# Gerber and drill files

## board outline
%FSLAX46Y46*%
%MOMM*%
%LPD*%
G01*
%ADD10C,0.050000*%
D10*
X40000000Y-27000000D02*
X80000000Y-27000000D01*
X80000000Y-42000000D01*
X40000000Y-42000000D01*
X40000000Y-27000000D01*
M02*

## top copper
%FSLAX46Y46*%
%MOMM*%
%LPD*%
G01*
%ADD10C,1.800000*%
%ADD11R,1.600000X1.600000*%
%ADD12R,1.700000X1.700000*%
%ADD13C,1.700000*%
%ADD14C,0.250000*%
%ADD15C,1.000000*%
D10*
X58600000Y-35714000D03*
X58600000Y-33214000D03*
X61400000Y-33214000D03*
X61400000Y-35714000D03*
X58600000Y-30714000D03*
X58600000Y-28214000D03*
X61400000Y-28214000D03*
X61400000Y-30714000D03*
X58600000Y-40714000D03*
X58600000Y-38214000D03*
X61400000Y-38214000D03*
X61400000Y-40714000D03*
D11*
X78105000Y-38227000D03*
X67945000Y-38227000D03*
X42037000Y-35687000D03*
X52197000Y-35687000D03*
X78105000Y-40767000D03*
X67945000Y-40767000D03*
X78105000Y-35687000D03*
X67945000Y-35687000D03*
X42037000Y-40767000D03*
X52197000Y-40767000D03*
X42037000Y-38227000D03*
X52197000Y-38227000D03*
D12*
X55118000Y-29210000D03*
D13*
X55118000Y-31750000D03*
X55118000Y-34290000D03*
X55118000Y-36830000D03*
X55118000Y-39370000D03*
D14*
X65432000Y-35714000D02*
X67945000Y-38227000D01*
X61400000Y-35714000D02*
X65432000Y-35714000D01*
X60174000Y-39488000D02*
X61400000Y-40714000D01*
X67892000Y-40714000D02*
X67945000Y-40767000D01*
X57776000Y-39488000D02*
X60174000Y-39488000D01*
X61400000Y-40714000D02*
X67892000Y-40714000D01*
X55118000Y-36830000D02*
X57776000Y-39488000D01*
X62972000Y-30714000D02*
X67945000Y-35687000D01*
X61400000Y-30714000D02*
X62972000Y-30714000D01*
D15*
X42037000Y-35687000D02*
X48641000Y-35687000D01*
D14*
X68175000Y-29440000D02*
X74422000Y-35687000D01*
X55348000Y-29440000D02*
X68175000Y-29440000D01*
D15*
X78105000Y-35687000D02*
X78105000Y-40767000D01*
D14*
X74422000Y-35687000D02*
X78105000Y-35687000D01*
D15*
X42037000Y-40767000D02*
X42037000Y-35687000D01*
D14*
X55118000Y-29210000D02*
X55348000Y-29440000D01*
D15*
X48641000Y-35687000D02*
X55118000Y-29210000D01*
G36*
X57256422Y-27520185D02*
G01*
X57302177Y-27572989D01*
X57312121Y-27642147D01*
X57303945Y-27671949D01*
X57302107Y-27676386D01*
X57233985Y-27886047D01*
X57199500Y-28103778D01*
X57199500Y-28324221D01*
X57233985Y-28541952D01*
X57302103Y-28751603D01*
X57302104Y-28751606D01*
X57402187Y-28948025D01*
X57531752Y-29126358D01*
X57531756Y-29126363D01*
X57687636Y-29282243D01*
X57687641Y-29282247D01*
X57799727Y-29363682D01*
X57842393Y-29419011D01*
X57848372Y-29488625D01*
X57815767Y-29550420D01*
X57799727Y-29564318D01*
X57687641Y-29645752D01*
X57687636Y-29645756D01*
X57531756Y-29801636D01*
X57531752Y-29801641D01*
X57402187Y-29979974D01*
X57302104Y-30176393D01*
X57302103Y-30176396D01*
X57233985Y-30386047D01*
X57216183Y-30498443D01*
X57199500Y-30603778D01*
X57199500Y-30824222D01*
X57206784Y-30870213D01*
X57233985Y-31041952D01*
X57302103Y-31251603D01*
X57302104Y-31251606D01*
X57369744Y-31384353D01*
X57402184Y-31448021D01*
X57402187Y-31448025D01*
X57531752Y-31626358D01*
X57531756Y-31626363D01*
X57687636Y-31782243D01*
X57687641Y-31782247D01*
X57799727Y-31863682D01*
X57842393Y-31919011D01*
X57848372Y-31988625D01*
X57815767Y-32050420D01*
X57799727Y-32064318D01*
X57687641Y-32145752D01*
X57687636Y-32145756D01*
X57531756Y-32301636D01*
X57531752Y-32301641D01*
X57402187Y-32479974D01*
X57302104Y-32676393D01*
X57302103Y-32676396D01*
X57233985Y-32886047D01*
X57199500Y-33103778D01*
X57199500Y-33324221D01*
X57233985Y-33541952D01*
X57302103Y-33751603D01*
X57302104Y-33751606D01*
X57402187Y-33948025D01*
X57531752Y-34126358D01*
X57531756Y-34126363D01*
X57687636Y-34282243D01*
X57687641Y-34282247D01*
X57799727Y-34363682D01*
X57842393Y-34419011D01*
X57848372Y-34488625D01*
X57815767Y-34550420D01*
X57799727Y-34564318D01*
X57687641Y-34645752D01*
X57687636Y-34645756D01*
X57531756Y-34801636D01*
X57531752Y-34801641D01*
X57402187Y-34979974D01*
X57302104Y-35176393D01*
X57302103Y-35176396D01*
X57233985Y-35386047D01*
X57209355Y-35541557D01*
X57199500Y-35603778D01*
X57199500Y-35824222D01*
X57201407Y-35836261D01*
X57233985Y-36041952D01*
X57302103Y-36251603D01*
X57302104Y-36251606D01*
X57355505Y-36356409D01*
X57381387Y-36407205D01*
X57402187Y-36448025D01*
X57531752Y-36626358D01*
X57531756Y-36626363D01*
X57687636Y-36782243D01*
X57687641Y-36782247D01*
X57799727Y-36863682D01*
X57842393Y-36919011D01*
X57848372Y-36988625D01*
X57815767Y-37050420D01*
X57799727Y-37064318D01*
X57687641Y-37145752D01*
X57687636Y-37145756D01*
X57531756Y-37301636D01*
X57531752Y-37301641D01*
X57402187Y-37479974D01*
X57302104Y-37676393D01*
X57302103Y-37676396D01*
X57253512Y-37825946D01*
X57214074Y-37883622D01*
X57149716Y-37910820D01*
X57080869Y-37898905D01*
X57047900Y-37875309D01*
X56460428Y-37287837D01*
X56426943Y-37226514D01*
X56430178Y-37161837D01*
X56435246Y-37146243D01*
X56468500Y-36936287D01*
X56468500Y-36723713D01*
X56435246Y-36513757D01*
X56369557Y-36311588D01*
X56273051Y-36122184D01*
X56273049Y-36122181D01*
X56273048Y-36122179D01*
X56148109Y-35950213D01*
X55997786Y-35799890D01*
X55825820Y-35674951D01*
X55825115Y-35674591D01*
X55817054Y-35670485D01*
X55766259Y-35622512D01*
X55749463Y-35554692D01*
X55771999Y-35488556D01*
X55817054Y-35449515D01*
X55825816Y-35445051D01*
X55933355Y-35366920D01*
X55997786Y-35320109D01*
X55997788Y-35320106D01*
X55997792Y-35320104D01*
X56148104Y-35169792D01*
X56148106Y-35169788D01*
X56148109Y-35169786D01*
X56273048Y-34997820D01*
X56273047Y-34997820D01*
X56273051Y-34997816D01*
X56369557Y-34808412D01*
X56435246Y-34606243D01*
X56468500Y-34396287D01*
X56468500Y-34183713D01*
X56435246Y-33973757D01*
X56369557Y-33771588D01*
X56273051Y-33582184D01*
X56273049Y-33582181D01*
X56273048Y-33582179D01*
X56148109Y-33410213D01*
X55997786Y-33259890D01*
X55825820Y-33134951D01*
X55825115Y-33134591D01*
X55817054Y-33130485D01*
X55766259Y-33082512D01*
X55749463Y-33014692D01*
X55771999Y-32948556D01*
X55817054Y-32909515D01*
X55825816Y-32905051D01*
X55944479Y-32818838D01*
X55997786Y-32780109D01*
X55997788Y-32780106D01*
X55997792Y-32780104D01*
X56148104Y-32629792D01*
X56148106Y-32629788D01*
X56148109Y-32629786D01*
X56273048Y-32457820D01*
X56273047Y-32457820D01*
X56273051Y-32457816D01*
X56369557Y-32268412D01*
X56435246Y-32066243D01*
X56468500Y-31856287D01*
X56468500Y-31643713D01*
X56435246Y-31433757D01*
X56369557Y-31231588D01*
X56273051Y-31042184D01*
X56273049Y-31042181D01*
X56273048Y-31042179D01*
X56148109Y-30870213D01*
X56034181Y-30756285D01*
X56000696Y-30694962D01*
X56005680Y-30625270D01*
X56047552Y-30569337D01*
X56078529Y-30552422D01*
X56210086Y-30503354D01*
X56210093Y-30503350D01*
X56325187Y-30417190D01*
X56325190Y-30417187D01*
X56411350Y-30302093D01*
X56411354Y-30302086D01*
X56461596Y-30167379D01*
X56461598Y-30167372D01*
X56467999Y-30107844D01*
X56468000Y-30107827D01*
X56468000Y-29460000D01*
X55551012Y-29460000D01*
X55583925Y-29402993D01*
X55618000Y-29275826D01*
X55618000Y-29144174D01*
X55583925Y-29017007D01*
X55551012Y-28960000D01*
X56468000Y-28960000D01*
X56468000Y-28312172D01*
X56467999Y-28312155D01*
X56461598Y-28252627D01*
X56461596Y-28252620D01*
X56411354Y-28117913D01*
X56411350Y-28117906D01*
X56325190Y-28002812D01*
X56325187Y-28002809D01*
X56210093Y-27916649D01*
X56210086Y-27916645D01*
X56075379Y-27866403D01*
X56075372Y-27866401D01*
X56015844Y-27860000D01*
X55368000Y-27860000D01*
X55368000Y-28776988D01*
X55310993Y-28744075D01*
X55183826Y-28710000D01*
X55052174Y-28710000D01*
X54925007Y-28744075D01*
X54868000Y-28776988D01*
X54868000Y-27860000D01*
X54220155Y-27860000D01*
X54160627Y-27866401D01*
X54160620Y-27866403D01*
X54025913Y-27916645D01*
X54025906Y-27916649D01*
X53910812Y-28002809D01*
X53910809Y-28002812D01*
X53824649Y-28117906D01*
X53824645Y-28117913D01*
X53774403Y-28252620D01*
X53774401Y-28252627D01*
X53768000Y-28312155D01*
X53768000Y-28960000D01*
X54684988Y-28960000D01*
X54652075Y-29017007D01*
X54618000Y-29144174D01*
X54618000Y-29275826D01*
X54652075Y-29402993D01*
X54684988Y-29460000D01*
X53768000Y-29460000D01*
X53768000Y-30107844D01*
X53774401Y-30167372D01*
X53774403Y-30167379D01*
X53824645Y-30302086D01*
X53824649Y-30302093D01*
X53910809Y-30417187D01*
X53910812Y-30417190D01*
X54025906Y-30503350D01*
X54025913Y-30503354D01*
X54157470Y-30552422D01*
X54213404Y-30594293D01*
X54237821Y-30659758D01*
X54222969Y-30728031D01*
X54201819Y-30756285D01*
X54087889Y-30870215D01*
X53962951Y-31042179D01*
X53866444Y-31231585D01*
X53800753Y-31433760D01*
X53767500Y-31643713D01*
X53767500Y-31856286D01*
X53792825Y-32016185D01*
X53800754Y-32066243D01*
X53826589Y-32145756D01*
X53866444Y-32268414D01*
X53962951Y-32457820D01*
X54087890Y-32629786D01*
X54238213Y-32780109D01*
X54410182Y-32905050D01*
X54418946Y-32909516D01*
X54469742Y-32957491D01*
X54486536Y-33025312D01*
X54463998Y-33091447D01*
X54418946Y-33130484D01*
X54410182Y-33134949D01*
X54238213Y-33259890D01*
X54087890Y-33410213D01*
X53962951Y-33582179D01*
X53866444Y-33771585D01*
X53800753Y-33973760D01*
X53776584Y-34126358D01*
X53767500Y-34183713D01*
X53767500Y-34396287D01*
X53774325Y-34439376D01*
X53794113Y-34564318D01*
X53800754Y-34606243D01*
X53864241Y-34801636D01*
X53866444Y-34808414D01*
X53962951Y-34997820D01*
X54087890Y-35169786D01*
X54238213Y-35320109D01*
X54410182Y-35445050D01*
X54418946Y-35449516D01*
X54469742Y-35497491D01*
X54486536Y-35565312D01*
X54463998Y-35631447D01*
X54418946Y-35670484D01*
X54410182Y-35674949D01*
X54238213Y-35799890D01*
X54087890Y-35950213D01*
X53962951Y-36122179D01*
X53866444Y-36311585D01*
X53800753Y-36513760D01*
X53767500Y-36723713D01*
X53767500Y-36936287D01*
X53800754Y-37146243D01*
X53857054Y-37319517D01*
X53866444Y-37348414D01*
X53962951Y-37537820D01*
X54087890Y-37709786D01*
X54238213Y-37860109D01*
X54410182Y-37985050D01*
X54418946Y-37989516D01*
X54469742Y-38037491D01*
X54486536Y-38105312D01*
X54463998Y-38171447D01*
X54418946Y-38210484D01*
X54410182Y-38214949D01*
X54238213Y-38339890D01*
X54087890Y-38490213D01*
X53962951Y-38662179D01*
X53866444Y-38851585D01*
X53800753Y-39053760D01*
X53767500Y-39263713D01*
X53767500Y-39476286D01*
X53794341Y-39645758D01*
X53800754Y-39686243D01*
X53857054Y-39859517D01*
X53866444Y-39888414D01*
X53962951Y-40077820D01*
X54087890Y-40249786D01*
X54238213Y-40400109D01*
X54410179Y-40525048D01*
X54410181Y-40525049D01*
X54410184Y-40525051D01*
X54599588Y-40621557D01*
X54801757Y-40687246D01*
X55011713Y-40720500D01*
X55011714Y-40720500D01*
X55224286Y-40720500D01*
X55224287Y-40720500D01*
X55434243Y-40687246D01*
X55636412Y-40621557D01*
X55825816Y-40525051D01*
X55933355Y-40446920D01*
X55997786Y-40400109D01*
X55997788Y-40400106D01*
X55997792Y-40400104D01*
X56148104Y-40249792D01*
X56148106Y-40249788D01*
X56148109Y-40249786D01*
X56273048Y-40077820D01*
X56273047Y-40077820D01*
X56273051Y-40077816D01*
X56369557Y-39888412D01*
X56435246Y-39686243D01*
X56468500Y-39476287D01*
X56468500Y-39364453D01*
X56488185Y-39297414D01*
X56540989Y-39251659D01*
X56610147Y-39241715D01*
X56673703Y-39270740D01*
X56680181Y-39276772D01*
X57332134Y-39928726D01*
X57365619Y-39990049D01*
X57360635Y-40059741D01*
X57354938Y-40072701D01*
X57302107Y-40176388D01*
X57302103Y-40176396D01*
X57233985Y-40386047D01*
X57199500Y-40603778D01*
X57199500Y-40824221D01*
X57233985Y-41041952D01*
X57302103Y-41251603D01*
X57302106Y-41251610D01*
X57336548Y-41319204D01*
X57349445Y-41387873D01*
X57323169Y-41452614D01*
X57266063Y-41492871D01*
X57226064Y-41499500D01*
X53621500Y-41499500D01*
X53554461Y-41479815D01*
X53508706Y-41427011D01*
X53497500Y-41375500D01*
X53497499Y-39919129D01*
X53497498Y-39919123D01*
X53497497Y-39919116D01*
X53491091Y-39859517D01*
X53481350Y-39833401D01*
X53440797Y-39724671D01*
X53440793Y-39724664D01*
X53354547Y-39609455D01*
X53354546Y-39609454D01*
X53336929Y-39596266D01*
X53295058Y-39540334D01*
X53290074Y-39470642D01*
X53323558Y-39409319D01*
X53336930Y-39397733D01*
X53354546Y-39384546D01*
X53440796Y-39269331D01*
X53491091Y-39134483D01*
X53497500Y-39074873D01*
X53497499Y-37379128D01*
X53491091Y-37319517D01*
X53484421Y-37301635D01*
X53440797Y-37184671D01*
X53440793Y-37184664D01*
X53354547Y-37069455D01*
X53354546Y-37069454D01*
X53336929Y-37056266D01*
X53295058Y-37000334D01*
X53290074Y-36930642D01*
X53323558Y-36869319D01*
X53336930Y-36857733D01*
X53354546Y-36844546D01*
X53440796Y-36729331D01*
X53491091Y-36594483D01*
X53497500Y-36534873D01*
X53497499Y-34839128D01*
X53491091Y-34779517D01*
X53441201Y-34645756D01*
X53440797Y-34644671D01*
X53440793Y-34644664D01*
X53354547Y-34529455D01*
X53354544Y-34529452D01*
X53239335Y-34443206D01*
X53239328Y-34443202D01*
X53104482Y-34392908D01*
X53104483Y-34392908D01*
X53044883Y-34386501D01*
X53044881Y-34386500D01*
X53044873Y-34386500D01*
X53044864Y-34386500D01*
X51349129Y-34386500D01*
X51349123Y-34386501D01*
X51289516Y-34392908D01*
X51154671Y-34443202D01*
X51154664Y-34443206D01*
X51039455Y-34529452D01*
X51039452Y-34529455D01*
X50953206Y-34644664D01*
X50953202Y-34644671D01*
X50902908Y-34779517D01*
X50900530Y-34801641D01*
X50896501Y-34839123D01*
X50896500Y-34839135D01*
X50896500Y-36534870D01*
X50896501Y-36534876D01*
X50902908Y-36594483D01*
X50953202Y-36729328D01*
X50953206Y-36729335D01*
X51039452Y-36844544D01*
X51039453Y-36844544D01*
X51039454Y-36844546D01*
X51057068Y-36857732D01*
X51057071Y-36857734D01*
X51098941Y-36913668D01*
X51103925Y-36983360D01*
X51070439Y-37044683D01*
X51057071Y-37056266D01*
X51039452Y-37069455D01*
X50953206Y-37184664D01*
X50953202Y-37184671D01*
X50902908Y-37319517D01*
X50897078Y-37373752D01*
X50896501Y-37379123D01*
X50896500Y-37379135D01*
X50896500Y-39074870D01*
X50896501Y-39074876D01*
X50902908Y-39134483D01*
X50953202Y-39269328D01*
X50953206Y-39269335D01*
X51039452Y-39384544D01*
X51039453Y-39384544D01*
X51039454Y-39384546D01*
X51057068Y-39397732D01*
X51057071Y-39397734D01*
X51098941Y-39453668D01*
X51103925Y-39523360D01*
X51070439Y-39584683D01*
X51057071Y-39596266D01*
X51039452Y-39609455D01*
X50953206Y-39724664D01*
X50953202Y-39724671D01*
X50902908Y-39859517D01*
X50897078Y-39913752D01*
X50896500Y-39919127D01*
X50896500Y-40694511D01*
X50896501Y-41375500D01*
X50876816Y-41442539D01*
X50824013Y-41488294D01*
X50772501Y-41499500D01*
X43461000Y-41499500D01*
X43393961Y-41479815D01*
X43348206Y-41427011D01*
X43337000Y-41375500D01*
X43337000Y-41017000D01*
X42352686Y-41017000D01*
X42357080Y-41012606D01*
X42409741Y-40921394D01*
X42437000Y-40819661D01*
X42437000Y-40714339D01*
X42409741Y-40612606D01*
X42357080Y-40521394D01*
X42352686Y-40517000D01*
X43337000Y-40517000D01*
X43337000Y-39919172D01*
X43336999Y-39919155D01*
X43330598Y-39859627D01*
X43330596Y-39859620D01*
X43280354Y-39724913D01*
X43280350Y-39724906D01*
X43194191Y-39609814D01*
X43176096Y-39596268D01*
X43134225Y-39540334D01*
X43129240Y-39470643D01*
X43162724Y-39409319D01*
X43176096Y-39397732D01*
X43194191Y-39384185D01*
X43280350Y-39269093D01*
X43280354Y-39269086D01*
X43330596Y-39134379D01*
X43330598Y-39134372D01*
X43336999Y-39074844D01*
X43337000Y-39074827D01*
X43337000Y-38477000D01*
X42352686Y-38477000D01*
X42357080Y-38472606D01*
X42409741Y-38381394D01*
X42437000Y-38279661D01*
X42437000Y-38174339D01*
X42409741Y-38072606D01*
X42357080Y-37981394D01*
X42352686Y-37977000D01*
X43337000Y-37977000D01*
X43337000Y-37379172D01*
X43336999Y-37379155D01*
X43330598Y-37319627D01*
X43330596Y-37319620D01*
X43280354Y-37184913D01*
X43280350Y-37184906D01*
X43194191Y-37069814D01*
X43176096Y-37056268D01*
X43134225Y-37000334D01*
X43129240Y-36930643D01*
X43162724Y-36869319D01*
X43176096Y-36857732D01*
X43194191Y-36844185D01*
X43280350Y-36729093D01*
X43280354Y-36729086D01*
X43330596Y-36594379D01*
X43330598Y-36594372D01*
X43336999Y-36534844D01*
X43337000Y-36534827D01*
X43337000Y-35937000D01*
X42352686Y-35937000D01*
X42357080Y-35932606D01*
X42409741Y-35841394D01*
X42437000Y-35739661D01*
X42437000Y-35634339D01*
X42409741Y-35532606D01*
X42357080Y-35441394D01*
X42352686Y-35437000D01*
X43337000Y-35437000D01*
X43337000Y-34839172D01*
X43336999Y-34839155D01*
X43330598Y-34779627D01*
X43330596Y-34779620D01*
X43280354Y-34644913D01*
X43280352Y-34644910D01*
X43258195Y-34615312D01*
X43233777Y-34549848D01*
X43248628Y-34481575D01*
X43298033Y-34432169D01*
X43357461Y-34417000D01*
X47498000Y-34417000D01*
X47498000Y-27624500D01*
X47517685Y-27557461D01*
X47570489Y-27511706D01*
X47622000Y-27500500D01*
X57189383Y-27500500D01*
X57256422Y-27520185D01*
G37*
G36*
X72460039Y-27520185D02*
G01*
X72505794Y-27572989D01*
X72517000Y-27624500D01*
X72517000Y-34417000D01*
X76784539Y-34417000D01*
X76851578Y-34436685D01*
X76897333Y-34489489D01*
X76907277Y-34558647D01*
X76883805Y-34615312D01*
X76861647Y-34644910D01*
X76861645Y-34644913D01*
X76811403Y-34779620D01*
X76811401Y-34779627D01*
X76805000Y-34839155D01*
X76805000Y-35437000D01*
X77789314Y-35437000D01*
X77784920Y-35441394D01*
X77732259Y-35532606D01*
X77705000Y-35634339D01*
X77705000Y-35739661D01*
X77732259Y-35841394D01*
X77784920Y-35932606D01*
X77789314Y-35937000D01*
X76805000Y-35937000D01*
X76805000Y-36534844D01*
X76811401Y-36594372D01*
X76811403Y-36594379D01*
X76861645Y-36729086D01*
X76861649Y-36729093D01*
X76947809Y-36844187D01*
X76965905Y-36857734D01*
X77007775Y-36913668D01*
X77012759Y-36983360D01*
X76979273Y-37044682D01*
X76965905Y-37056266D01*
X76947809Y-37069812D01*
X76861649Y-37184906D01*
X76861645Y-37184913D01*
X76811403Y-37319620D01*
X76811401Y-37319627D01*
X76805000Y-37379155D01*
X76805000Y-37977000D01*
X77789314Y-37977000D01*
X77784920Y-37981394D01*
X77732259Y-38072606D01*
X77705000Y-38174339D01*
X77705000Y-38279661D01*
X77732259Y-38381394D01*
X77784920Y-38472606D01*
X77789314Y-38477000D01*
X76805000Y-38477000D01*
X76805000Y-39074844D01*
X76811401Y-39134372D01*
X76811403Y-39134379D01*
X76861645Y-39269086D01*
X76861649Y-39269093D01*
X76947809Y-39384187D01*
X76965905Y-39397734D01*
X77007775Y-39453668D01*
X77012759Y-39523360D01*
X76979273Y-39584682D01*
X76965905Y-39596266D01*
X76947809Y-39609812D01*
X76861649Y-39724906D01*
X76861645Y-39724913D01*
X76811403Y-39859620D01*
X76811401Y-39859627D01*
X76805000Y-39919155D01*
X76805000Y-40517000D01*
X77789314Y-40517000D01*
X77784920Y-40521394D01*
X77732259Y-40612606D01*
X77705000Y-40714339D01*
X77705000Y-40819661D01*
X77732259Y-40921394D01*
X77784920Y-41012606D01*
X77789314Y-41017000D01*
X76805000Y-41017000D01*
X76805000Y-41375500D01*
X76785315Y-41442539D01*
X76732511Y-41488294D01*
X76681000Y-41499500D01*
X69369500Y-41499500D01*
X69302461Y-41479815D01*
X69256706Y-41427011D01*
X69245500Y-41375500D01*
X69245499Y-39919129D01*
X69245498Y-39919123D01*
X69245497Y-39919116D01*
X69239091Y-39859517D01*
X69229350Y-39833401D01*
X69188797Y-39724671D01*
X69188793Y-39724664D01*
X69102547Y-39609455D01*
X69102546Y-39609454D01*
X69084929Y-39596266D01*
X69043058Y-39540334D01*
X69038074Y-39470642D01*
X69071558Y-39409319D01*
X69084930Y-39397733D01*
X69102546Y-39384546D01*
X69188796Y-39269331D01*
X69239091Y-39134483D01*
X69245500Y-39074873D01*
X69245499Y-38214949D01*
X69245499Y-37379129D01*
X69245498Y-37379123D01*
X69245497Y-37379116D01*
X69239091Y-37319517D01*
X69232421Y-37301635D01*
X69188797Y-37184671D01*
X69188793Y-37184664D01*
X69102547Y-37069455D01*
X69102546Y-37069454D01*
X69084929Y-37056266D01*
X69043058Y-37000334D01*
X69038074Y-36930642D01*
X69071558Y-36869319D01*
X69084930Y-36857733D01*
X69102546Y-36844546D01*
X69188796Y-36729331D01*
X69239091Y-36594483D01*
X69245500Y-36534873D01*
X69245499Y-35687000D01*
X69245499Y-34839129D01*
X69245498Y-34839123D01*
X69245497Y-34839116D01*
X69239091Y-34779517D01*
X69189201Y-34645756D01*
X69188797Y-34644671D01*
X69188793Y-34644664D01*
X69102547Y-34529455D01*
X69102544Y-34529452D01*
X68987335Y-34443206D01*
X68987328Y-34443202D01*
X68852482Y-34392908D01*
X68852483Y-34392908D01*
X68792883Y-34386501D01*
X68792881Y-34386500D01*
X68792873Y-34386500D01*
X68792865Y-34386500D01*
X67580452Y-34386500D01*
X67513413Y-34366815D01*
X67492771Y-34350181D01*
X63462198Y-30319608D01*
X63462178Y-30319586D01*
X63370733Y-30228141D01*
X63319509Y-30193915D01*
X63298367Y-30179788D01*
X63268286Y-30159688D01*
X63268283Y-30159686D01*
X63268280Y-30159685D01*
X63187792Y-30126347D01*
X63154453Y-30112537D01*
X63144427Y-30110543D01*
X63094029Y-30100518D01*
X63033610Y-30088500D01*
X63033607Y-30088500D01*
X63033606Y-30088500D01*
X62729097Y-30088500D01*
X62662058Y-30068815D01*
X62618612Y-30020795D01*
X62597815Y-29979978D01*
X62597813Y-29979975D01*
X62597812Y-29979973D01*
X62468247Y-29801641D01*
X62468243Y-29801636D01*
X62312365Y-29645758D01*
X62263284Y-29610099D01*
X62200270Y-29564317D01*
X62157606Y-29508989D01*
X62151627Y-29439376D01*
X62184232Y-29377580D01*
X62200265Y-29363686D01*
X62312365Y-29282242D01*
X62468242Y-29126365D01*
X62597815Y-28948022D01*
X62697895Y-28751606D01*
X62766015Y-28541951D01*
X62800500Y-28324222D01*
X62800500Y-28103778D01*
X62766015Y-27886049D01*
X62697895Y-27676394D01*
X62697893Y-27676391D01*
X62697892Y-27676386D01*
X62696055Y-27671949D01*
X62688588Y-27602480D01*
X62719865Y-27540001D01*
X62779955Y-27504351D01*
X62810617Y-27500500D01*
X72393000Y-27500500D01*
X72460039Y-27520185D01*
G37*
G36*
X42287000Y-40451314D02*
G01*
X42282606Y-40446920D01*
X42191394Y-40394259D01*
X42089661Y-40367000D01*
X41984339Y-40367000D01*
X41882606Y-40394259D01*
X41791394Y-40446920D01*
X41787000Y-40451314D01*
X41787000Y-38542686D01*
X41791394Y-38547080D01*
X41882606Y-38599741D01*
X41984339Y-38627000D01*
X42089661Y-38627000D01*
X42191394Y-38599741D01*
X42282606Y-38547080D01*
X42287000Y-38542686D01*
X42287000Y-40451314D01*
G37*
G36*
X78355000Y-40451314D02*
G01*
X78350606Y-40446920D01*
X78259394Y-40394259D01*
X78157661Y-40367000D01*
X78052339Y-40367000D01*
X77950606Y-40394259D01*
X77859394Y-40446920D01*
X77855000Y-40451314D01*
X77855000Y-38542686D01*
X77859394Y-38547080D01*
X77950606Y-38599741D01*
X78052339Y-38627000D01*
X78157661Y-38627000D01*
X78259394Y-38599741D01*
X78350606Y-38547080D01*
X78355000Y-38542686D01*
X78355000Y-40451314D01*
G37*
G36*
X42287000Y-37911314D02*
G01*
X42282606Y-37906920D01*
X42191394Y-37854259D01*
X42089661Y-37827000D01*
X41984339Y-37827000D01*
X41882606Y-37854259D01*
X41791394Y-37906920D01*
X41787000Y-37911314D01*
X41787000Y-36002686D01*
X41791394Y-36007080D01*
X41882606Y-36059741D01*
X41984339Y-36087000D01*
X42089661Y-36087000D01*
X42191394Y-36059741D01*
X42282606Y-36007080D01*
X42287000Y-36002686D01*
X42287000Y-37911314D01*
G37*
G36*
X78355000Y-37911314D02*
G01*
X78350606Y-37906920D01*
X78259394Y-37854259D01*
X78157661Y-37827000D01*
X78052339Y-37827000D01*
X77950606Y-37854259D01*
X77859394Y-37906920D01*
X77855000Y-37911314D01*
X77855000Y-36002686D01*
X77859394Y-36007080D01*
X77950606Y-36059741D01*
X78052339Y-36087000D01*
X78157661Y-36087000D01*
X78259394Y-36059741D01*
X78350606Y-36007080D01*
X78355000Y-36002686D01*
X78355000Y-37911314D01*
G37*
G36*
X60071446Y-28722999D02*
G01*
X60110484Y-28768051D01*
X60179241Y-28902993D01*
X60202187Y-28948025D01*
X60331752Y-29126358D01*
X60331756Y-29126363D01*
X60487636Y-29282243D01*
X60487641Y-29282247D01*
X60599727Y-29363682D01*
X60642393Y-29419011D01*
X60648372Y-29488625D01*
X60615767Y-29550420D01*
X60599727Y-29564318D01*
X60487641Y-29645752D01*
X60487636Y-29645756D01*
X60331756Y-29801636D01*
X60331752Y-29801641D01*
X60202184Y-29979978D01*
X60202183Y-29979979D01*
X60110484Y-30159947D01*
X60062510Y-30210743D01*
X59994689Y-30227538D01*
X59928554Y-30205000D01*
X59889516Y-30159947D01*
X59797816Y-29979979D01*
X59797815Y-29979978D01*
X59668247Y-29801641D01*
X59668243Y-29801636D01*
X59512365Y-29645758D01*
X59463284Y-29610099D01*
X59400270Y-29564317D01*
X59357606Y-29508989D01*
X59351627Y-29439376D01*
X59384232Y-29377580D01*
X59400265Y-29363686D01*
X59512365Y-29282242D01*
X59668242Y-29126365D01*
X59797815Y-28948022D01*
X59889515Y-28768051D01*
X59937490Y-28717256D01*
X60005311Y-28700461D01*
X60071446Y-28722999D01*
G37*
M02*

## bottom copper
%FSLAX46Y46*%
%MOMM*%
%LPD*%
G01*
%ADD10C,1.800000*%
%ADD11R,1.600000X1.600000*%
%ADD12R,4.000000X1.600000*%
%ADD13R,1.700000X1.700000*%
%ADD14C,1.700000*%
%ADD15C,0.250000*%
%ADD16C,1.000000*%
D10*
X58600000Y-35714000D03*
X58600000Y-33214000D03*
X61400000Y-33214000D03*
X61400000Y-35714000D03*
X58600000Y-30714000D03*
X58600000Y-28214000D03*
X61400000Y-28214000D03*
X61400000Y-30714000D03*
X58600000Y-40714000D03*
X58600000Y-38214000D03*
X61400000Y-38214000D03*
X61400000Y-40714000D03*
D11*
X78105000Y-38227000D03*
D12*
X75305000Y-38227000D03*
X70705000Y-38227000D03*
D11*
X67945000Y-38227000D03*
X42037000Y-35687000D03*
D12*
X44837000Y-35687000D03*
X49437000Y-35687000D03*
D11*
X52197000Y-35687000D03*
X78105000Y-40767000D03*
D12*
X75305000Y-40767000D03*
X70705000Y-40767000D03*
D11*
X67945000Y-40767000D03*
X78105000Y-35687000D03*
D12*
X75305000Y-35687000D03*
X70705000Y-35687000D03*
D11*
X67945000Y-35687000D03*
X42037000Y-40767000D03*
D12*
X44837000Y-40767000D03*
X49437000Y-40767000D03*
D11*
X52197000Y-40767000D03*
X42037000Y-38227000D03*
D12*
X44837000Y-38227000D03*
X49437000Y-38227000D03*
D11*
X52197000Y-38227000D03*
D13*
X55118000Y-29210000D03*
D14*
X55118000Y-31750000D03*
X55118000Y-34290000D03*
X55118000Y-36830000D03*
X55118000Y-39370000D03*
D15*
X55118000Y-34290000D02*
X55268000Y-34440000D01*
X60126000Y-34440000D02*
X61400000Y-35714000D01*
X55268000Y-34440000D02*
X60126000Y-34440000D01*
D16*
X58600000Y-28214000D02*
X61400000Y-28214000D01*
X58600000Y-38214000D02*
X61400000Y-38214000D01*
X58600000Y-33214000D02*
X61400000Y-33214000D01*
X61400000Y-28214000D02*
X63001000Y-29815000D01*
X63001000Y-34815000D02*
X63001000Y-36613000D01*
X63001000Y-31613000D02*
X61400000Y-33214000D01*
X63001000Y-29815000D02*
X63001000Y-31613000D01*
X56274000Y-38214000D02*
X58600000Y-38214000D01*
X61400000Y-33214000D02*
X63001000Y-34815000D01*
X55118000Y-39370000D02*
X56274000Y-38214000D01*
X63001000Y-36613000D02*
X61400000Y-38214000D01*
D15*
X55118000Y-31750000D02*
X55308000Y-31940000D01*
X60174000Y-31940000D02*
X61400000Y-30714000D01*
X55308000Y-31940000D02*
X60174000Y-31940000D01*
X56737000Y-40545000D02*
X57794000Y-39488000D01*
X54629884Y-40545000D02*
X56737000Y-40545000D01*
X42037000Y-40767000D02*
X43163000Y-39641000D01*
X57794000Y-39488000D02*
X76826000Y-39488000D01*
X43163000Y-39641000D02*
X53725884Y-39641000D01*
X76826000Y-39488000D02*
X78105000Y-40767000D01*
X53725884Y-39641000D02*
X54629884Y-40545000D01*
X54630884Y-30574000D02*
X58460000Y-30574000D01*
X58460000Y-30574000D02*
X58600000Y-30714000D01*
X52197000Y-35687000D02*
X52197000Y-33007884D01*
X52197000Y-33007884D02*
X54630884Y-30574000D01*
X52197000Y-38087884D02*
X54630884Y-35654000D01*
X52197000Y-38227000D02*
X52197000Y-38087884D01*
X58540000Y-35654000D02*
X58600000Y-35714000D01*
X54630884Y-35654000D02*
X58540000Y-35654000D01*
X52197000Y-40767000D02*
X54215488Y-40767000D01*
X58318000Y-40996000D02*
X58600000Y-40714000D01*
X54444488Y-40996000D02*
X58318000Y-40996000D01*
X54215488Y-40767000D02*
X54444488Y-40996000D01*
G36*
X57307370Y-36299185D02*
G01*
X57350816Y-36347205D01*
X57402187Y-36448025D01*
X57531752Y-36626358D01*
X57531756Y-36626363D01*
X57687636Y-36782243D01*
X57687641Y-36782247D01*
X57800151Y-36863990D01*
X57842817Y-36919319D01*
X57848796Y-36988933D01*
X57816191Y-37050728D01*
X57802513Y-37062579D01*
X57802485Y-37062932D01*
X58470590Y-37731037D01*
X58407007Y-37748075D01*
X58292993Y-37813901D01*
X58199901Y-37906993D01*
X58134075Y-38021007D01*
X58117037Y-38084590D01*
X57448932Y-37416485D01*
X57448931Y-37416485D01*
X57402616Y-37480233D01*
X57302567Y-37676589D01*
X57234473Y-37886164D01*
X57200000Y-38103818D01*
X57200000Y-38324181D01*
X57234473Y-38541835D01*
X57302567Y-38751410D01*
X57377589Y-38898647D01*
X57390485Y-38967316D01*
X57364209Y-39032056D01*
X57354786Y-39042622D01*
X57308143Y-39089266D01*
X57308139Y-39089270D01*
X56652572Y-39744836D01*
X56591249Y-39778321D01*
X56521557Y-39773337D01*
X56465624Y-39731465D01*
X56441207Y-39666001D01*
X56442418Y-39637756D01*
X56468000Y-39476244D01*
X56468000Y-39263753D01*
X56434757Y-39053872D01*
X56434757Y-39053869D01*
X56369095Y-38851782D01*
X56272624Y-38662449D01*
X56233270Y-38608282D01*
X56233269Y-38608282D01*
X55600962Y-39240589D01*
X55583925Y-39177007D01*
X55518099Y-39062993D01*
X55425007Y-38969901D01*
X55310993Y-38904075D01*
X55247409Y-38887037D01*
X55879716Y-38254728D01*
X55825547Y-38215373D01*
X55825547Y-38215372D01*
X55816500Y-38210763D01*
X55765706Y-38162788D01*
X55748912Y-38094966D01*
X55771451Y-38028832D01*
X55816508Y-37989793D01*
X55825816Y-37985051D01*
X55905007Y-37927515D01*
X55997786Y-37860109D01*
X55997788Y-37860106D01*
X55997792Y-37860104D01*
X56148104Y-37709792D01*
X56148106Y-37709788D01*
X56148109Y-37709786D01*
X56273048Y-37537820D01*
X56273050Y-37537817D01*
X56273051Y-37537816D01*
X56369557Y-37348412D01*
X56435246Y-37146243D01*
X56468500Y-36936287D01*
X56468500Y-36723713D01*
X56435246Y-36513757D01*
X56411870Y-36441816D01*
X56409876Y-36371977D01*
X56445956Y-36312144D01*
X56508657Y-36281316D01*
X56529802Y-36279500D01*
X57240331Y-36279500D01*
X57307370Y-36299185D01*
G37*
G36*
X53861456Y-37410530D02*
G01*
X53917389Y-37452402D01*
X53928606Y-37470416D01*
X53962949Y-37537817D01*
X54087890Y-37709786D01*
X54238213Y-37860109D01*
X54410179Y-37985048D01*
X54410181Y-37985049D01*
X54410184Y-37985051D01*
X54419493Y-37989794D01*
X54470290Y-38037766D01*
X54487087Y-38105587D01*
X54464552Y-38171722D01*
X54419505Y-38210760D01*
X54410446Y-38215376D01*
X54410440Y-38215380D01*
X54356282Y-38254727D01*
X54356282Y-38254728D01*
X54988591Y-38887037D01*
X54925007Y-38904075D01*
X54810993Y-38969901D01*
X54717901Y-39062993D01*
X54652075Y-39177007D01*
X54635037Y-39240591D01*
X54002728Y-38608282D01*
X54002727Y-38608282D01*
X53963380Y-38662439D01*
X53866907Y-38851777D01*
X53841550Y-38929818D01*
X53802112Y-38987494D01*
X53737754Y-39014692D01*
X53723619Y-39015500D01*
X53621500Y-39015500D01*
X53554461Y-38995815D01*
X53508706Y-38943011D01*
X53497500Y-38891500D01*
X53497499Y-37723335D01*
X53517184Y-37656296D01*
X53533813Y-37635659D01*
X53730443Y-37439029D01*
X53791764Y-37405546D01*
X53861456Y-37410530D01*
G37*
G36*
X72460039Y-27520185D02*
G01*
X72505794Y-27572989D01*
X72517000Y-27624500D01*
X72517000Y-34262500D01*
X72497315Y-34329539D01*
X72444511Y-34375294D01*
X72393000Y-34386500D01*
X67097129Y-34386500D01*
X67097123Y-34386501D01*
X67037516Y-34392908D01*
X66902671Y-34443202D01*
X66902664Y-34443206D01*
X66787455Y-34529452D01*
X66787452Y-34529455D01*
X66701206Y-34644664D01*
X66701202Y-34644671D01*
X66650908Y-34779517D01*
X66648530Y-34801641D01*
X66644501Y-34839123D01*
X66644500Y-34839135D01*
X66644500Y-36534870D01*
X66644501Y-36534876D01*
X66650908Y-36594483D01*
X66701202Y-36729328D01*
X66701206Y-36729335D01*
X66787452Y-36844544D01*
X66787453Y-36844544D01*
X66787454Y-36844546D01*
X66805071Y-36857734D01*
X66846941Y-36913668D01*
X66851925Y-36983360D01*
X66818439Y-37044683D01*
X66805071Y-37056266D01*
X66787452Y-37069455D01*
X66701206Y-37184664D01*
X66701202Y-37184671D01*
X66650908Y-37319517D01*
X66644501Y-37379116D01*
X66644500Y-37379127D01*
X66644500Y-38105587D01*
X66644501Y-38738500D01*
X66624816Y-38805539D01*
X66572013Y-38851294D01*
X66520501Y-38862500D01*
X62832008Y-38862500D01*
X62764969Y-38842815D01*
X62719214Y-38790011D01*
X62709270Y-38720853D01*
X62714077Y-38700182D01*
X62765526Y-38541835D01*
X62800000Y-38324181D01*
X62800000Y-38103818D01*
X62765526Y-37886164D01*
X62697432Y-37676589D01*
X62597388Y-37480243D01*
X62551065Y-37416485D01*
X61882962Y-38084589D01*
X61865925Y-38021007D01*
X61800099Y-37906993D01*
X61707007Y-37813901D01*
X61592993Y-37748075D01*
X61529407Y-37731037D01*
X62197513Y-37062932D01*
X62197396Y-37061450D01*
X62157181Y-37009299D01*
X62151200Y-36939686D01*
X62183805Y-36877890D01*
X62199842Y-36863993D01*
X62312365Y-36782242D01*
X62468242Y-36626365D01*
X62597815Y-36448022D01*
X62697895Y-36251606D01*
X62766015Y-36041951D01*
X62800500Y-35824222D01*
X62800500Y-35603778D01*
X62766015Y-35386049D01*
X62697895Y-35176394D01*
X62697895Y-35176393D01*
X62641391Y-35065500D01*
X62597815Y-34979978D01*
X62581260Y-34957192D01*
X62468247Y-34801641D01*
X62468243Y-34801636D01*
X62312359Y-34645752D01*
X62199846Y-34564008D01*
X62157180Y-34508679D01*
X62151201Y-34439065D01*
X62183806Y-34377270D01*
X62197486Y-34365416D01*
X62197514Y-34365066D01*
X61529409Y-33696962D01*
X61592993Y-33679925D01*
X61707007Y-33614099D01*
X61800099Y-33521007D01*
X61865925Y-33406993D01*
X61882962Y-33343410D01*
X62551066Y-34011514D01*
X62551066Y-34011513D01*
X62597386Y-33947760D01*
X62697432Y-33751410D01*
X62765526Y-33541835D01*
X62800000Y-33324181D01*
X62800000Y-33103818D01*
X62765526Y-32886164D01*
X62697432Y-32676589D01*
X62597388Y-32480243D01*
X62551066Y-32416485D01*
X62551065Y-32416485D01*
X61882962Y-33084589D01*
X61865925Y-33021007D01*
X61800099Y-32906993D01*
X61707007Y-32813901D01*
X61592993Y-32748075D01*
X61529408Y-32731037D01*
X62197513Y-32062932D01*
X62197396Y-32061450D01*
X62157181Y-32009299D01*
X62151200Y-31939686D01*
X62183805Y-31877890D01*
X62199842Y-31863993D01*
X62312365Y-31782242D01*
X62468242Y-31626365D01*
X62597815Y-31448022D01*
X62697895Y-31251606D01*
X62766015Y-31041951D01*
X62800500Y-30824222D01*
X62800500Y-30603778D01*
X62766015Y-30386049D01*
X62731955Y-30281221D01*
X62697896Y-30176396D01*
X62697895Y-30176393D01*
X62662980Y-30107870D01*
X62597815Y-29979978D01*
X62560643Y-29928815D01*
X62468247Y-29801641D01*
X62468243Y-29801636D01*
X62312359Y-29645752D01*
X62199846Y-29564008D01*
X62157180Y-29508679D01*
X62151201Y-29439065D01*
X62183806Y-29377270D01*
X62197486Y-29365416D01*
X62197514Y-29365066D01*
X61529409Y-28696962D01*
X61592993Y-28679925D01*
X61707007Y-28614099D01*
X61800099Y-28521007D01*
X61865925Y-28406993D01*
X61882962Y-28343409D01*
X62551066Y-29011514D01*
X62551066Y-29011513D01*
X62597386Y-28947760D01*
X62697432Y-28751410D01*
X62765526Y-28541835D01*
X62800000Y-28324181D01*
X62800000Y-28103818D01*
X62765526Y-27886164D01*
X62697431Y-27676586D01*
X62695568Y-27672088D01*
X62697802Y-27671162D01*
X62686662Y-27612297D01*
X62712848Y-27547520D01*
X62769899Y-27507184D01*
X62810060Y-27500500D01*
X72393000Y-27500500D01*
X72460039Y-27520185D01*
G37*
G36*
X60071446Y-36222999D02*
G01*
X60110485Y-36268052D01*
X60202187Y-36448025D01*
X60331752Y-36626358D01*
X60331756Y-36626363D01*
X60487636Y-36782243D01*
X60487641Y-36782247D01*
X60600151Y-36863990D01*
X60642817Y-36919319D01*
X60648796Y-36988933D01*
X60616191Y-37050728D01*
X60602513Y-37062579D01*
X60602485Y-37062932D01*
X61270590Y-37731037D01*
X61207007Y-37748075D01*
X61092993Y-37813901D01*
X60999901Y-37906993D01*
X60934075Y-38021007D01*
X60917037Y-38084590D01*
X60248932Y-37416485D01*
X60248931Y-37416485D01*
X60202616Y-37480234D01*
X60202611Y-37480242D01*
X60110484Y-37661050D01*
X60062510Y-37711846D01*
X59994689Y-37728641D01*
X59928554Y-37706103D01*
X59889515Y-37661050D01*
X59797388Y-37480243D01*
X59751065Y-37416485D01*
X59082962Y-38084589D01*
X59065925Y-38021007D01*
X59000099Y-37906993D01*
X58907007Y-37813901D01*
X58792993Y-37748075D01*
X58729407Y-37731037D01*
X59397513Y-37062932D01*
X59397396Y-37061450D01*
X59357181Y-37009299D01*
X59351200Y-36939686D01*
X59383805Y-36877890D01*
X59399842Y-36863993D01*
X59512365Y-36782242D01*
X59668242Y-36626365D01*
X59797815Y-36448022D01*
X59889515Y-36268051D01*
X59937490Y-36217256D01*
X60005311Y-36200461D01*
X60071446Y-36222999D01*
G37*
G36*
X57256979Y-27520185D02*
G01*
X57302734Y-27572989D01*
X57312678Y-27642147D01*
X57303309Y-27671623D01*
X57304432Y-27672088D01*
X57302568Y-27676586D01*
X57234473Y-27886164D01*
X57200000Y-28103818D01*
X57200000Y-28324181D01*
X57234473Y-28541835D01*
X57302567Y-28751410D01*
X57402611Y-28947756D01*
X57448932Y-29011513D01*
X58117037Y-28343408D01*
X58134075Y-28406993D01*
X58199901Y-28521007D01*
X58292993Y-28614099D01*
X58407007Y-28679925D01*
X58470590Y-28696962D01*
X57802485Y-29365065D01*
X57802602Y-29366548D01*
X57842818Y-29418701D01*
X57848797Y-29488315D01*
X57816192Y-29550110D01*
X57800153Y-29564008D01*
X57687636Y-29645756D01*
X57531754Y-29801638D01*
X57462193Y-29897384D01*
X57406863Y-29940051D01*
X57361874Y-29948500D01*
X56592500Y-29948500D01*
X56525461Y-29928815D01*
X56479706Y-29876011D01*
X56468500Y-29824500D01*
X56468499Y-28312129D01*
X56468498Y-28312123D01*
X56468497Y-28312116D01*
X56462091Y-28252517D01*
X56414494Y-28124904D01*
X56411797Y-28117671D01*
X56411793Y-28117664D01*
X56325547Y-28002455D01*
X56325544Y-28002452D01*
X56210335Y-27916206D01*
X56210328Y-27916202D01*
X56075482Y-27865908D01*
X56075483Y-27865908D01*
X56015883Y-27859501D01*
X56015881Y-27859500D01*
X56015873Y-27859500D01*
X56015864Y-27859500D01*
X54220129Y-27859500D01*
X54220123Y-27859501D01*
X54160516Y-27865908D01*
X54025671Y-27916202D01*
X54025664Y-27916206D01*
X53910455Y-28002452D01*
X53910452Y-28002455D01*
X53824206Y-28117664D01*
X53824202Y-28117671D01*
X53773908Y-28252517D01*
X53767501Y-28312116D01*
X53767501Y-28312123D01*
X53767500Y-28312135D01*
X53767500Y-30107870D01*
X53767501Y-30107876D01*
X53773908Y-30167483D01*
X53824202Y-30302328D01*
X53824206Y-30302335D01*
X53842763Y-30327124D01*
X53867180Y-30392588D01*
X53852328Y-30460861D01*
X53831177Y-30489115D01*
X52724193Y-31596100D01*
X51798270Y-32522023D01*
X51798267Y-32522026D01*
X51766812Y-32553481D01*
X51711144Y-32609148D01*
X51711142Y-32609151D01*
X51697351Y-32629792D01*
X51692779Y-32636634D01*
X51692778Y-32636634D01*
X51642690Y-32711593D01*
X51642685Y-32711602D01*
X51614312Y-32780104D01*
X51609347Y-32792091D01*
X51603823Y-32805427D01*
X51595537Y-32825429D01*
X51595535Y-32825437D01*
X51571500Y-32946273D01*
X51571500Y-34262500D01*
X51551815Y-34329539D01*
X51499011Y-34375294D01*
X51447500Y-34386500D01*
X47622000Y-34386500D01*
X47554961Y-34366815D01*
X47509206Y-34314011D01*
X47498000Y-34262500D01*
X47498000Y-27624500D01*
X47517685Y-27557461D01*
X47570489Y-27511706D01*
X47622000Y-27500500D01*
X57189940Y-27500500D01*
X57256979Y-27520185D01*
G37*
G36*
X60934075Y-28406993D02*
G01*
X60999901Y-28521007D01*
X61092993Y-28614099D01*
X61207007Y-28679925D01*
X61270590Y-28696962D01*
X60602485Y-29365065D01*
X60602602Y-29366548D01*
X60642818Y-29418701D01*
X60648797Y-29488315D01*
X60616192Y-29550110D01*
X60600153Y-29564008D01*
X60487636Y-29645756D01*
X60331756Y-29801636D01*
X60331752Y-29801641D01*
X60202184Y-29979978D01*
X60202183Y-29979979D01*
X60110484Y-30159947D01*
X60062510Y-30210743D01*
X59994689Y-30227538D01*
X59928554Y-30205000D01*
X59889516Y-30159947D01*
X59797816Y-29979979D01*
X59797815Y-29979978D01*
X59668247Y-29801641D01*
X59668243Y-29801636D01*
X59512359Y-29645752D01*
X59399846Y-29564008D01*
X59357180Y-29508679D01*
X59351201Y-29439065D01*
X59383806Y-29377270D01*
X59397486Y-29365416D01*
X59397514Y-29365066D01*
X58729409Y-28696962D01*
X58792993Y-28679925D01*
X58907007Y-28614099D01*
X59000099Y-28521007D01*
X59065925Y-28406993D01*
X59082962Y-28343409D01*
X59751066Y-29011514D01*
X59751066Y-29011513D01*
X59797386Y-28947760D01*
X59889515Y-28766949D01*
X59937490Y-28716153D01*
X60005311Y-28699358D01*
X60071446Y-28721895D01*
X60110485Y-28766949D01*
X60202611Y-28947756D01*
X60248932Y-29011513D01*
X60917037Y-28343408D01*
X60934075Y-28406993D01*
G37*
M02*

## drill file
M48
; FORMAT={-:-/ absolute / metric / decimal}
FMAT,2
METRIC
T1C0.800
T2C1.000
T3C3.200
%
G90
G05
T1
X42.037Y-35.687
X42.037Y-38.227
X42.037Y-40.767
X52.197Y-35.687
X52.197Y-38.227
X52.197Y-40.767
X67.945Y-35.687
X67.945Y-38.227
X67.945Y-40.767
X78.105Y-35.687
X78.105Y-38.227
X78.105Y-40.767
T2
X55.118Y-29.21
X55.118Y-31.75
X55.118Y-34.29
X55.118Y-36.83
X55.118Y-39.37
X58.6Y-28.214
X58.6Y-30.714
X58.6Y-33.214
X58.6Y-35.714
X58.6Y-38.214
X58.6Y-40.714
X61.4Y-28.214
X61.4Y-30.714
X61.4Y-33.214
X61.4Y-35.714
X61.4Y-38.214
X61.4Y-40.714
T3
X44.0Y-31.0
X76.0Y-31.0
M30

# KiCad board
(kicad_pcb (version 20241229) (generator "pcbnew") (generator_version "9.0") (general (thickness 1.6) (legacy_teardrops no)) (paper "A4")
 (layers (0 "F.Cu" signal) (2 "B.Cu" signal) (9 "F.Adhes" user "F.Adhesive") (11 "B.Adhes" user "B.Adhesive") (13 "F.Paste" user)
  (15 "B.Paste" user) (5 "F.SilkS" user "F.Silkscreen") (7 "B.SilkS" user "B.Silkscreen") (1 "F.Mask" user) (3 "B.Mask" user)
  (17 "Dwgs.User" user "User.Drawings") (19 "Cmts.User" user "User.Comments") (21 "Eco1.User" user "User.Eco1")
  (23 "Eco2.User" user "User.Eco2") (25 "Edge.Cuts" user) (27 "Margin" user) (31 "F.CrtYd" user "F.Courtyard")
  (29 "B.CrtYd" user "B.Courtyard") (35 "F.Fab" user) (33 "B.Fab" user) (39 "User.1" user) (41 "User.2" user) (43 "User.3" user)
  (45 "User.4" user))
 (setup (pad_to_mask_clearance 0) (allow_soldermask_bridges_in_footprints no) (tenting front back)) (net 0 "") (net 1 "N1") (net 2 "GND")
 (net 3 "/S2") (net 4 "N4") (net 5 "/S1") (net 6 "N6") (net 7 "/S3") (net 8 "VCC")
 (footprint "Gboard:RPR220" (layer "F.Cu") (at 60 34.464)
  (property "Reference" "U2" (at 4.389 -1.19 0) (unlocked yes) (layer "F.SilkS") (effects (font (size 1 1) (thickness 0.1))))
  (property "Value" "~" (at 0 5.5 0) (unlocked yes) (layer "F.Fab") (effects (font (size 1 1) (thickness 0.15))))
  (pad "1" thru_hole circle (at -1.4 1.25) (size 1.8 1.8) (drill 1) (layers "*.Cu" "*.Mask") (remove_unused_layers no) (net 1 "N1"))
  (pad "2" thru_hole circle (at -1.4 -1.25) (size 1.8 1.8) (drill 1) (layers "*.Cu" "*.Mask") (remove_unused_layers no) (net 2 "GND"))
  (pad "3" thru_hole circle (at 1.4 -1.25) (size 1.8 1.8) (drill 1) (layers "*.Cu" "*.Mask") (remove_unused_layers no) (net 2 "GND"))
  (pad "4" thru_hole circle (at 1.4 1.25) (size 1.8 1.8) (drill 1) (layers "*.Cu" "*.Mask") (remove_unused_layers no) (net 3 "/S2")))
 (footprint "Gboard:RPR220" (layer "F.Cu") (at 60 29.464)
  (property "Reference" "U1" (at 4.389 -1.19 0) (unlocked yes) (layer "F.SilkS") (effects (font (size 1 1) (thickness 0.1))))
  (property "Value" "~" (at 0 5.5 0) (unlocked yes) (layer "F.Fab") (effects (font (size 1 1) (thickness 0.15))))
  (pad "1" thru_hole circle (at -1.4 1.25) (size 1.8 1.8) (drill 1) (layers "*.Cu" "*.Mask") (remove_unused_layers no) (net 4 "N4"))
  (pad "2" thru_hole circle (at -1.4 -1.25) (size 1.8 1.8) (drill 1) (layers "*.Cu" "*.Mask") (remove_unused_layers no) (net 2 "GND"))
  (pad "3" thru_hole circle (at 1.4 -1.25) (size 1.8 1.8) (drill 1) (layers "*.Cu" "*.Mask") (remove_unused_layers no) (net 2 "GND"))
  (pad "4" thru_hole circle (at 1.4 1.25) (size 1.8 1.8) (drill 1) (layers "*.Cu" "*.Mask") (remove_unused_layers no) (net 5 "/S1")))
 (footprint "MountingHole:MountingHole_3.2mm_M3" (layer "F.Cu") (at 76 31)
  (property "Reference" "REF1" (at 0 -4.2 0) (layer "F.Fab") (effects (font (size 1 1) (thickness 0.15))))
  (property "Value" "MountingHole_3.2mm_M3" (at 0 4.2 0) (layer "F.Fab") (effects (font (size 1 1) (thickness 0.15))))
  (pad "" np_thru_hole circle (at 0 0) (size 3.2 3.2) (drill 3.2) (layers "*.Cu" "*.Mask")))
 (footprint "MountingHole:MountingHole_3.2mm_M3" (layer "F.Cu") (at 44 31)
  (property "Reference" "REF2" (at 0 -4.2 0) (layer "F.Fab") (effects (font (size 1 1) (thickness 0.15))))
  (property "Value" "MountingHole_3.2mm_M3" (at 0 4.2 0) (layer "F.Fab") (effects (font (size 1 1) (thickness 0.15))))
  (pad "" np_thru_hole circle (at 0 0) (size 3.2 3.2) (drill 3.2) (layers "*.Cu" "*.Mask")))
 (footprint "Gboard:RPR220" (layer "F.Cu") (at 60 39.464)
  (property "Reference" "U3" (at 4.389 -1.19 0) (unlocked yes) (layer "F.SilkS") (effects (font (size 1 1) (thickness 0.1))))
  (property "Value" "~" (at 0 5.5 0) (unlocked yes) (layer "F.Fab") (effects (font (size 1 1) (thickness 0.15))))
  (pad "1" thru_hole circle (at -1.4 1.25) (size 1.8 1.8) (drill 1) (layers "*.Cu" "*.Mask") (remove_unused_layers no) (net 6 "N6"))
  (pad "2" thru_hole circle (at -1.4 -1.25) (size 1.8 1.8) (drill 1) (layers "*.Cu" "*.Mask") (remove_unused_layers no) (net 2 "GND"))
  (pad "3" thru_hole circle (at 1.4 -1.25) (size 1.8 1.8) (drill 1) (layers "*.Cu" "*.Mask") (remove_unused_layers no) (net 2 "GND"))
  (pad "4" thru_hole circle (at 1.4 1.25) (size 1.8 1.8) (drill 1) (layers "*.Cu" "*.Mask") (remove_unused_layers no) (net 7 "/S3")))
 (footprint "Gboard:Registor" (layer "B.Cu") (at 78.105 38.227 180)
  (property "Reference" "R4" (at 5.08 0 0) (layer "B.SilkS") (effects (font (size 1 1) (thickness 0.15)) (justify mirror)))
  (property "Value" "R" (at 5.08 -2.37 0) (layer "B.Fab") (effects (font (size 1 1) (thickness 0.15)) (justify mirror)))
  (pad "1" thru_hole rect (at 0 0 180) (size 1.6 1.6) (drill 0.8) (layers "*.Cu" "*.Mask") (remove_unused_layers no) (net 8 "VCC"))
  (pad "1" smd rect (at 2.8 0 180) (size 4 1.6) (layers "B.Cu" "B.Mask" "B.Paste") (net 8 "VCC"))
  (pad "2" smd rect (at 7.4 0 180) (size 4 1.6) (layers "B.Cu" "B.Mask" "B.Paste") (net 3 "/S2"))
  (pad "2" thru_hole rect (at 10.16 0 180) (size 1.6 1.6) (drill 0.8) (layers "*.Cu" "*.Mask") (remove_unused_layers no) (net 3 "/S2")))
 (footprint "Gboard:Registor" (layer "B.Cu") (at 42.037 35.687)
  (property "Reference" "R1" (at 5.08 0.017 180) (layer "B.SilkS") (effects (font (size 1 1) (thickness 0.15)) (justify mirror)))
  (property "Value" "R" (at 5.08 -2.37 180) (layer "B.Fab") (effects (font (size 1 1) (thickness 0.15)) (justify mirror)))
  (pad "1" thru_hole rect (at 0 0) (size 1.6 1.6) (drill 0.8) (layers "*.Cu" "*.Mask") (remove_unused_layers no) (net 8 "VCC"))
  (pad "1" smd rect (at 2.8 0) (size 4 1.6) (layers "B.Cu" "B.Mask" "B.Paste") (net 8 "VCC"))
  (pad "2" smd rect (at 7.4 0) (size 4 1.6) (layers "B.Cu" "B.Mask" "B.Paste") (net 4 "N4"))
  (pad "2" thru_hole rect (at 10.16 0) (size 1.6 1.6) (drill 0.8) (layers "*.Cu" "*.Mask") (remove_unused_layers no) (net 4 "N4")))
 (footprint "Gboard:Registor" (layer "B.Cu") (at 78.105 40.767 180)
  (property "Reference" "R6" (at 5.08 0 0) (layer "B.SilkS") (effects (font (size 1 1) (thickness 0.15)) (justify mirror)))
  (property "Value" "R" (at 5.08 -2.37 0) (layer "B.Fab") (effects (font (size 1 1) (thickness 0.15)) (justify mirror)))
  (pad "1" thru_hole rect (at 0 0 180) (size 1.6 1.6) (drill 0.8) (layers "*.Cu" "*.Mask") (remove_unused_layers no) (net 8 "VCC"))
  (pad "1" smd rect (at 2.8 0 180) (size 4 1.6) (layers "B.Cu" "B.Mask" "B.Paste") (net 8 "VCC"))
  (pad "2" smd rect (at 7.4 0 180) (size 4 1.6) (layers "B.Cu" "B.Mask" "B.Paste") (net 7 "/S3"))
  (pad "2" thru_hole rect (at 10.16 0 180) (size 1.6 1.6) (drill 0.8) (layers "*.Cu" "*.Mask") (remove_unused_layers no) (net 7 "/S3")))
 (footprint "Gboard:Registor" (layer "B.Cu") (at 78.105 35.687 180)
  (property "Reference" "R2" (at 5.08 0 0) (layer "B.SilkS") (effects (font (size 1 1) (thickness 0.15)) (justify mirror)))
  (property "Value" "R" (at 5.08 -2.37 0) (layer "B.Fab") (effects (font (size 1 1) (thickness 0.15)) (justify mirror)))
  (pad "1" thru_hole rect (at 0 0 180) (size 1.6 1.6) (drill 0.8) (layers "*.Cu" "*.Mask") (remove_unused_layers no) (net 8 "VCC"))
  (pad "1" smd rect (at 2.8 0 180) (size 4 1.6) (layers "B.Cu" "B.Mask" "B.Paste") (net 8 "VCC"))
  (pad "2" smd rect (at 7.4 0 180) (size 4 1.6) (layers "B.Cu" "B.Mask" "B.Paste") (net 5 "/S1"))
  (pad "2" thru_hole rect (at 10.16 0 180) (size 1.6 1.6) (drill 0.8) (layers "*.Cu" "*.Mask") (remove_unused_layers no) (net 5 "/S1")))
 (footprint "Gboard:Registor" (layer "B.Cu") (at 42.037 40.767)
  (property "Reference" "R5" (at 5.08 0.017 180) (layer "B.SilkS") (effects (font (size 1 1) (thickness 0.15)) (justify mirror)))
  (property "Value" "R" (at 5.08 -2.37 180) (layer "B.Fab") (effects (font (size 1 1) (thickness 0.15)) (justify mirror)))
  (pad "1" thru_hole rect (at 0 0) (size 1.6 1.6) (drill 0.8) (layers "*.Cu" "*.Mask") (remove_unused_layers no) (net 8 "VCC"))
  (pad "1" smd rect (at 2.8 0) (size 4 1.6) (layers "B.Cu" "B.Mask" "B.Paste") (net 8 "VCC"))
  (pad "2" smd rect (at 7.4 0) (size 4 1.6) (layers "B.Cu" "B.Mask" "B.Paste") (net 6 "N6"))
  (pad "2" thru_hole rect (at 10.16 0) (size 1.6 1.6) (drill 0.8) (layers "*.Cu" "*.Mask") (remove_unused_layers no) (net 6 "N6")))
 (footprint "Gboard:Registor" (layer "B.Cu") (at 42.037 38.227)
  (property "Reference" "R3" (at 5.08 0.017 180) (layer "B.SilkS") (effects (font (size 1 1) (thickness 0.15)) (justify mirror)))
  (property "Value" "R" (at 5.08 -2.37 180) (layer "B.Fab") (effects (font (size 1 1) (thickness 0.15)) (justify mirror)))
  (pad "1" thru_hole rect (at 0 0) (size 1.6 1.6) (drill 0.8) (layers "*.Cu" "*.Mask") (remove_unused_layers no) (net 8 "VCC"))
  (pad "1" smd rect (at 2.8 0) (size 4 1.6) (layers "B.Cu" "B.Mask" "B.Paste") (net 8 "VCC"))
  (pad "2" smd rect (at 7.4 0) (size 4 1.6) (layers "B.Cu" "B.Mask" "B.Paste") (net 1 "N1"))
  (pad "2" thru_hole rect (at 10.16 0) (size 1.6 1.6) (drill 0.8) (layers "*.Cu" "*.Mask") (remove_unused_layers no) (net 1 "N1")))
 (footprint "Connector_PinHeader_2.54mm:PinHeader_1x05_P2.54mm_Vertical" (layer "B.Cu") (at 55.118 29.21 180)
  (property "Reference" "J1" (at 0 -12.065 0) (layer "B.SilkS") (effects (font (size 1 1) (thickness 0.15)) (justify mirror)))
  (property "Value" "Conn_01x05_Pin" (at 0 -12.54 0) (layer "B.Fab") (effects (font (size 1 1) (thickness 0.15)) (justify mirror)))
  (pad "1" thru_hole rect (at 0 0 180) (size 1.7 1.7) (drill 1) (layers "*.Cu" "*.Mask") (remove_unused_layers no) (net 8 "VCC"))
  (pad "2" thru_hole circle (at 0 -2.54 180) (size 1.7 1.7) (drill 1) (layers "*.Cu" "*.Mask") (remove_unused_layers no) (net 5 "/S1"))
  (pad "3" thru_hole circle (at 0 -5.08 180) (size 1.7 1.7) (drill 1) (layers "*.Cu" "*.Mask") (remove_unused_layers no) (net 3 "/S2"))
  (pad "4" thru_hole circle (at 0 -7.62 180) (size 1.7 1.7) (drill 1) (layers "*.Cu" "*.Mask") (remove_unused_layers no) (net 7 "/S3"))
  (pad "5" thru_hole circle (at 0 -10.16 180) (size 1.7 1.7) (drill 1) (layers "*.Cu" "*.Mask") (remove_unused_layers no) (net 2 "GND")))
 (gr_rect (start 40 27) (end 80 42) (stroke (width 0.05) (type default)) (fill no) (layer "Edge.Cuts"))
 (segment (start 65.432 35.714) (end 67.945 38.227) (width 0.25) (layer "F.Cu") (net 3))
 (segment (start 61.4 35.714) (end 65.432 35.714) (width 0.25) (layer "F.Cu") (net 3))
 (segment (start 55.118 34.29) (end 55.268 34.44) (width 0.25) (layer "B.Cu") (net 3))
 (segment (start 60.126 34.44) (end 61.4 35.714) (width 0.25) (layer "B.Cu") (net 3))
 (segment (start 55.268 34.44) (end 60.126 34.44) (width 0.25) (layer "B.Cu") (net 3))
 (segment (start 58.6 28.214) (end 61.4 28.214) (width 1) (layer "B.Cu") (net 2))
 (segment (start 58.6 38.214) (end 61.4 38.214) (width 1) (layer "B.Cu") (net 2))
 (segment (start 58.6 33.214) (end 61.4 33.214) (width 1) (layer "B.Cu") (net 2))
 (segment (start 61.4 28.214) (end 63.001 29.815) (width 1) (layer "B.Cu") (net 2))
 (segment (start 63.001 34.815) (end 63.001 36.613) (width 1) (layer "B.Cu") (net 2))
 (segment (start 63.001 31.613) (end 61.4 33.214) (width 1) (layer "B.Cu") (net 2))
 (segment (start 63.001 29.815) (end 63.001 31.613) (width 1) (layer "B.Cu") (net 2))
 (segment (start 56.274 38.214) (end 58.6 38.214) (width 1) (layer "B.Cu") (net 2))
 (segment (start 61.4 33.214) (end 63.001 34.815) (width 1) (layer "B.Cu") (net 2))
 (segment (start 55.118 39.37) (end 56.274 38.214) (width 1) (layer "B.Cu") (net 2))
 (segment (start 63.001 36.613) (end 61.4 38.214) (width 1) (layer "B.Cu") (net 2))
 (segment (start 60.174 39.488) (end 61.4 40.714) (width 0.25) (layer "F.Cu") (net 7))
 (segment (start 67.892 40.714) (end 67.945 40.767) (width 0.25) (layer "F.Cu") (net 7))
 (segment (start 57.776 39.488) (end 60.174 39.488) (width 0.25) (layer "F.Cu") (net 7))
 (segment (start 61.4 40.714) (end 67.892 40.714) (width 0.25) (layer "F.Cu") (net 7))
 (segment (start 55.118 36.83) (end 57.776 39.488) (width 0.25) (layer "F.Cu") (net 7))
 (segment (start 62.972 30.714) (end 67.945 35.687) (width 0.25) (layer "F.Cu") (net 5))
 (segment (start 61.4 30.714) (end 62.972 30.714) (width 0.25) (layer "F.Cu") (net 5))
 (segment (start 55.118 31.75) (end 55.308 31.94) (width 0.25) (layer "B.Cu") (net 5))
 (segment (start 60.174 31.94) (end 61.4 30.714) (width 0.25) (layer "B.Cu") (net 5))
 (segment (start 55.308 31.94) (end 60.174 31.94) (width 0.25) (layer "B.Cu") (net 5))
 (segment (start 42.037 35.687) (end 48.641 35.687) (width 1) (layer "F.Cu") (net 8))
 (segment (start 68.175 29.44) (end 74.422 35.687) (width 0.25) (layer "F.Cu") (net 8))
 (segment (start 55.348 29.44) (end 68.175 29.44) (width 0.25) (layer "F.Cu") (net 8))
 (segment (start 78.105 35.687) (end 78.105 40.767) (width 1) (layer "F.Cu") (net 8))
 (segment (start 74.422 35.687) (end 78.105 35.687) (width 0.25) (layer "F.Cu") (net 8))
 (segment (start 42.037 40.767) (end 42.037 35.687) (width 1) (layer "F.Cu") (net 8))
 (segment (start 55.118 29.21) (end 55.348 29.44) (width 0.25) (layer "F.Cu") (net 8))
 (segment (start 48.641 35.687) (end 55.118 29.21) (width 1) (layer "F.Cu") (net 8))
 (segment (start 56.737 40.545) (end 57.794 39.488) (width 0.25) (layer "B.Cu") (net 8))
 (segment (start 54.629884 40.545) (end 56.737 40.545) (width 0.25) (layer "B.Cu") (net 8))
 (segment (start 42.037 40.767) (end 43.163 39.641) (width 0.25) (layer "B.Cu") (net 8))
 (segment (start 57.794 39.488) (end 76.826 39.488) (width 0.25) (layer "B.Cu") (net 8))
 (segment (start 43.163 39.641) (end 53.725884 39.641) (width 0.25) (layer "B.Cu") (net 8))
 (segment (start 76.826 39.488) (end 78.105 40.767) (width 0.25) (layer "B.Cu") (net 8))
 (segment (start 53.725884 39.641) (end 54.629884 40.545) (width 0.25) (layer "B.Cu") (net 8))
 (segment (start 54.630884 30.574) (end 58.46 30.574) (width 0.25) (layer "B.Cu") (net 4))
 (segment (start 58.46 30.574) (end 58.6 30.714) (width 0.25) (layer "B.Cu") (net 4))
 (segment (start 52.197 35.687) (end 52.197 33.007884) (width 0.25) (layer "B.Cu") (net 4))
 (segment (start 52.197 33.007884) (end 54.630884 30.574) (width 0.25) (layer "B.Cu") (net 4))
 (segment (start 52.197 38.087884) (end 54.630884 35.654) (width 0.25) (layer "B.Cu") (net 1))
 (segment (start 52.197 38.227) (end 52.197 38.087884) (width 0.25) (layer "B.Cu") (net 1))
 (segment (start 58.54 35.654) (end 58.6 35.714) (width 0.25) (layer "B.Cu") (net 1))
 (segment (start 54.630884 35.654) (end 58.54 35.654) (width 0.25) (layer "B.Cu") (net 1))
 (segment (start 52.197 40.767) (end 54.215488 40.767) (width 0.25) (layer "B.Cu") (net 6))
 (segment (start 58.318 40.996) (end 58.6 40.714) (width 0.25) (layer "B.Cu") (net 6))
 (segment (start 54.444488 40.996) (end 58.318 40.996) (width 0.25) (layer "B.Cu") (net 6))
 (segment (start 54.215488 40.767) (end 54.444488 40.996) (width 0.25) (layer "B.Cu") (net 6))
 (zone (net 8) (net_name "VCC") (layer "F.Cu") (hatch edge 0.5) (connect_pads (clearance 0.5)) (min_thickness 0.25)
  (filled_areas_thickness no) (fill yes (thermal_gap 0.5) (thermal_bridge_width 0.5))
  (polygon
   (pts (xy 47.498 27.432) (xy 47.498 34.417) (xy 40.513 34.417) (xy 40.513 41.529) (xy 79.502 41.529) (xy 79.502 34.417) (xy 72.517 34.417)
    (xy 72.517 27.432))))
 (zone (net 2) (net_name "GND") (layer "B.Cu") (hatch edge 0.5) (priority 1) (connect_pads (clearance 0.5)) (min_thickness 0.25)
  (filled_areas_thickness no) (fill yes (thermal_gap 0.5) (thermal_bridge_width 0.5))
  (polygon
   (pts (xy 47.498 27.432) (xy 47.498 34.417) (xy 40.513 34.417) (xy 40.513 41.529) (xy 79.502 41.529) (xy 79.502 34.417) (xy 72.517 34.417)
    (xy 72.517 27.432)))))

